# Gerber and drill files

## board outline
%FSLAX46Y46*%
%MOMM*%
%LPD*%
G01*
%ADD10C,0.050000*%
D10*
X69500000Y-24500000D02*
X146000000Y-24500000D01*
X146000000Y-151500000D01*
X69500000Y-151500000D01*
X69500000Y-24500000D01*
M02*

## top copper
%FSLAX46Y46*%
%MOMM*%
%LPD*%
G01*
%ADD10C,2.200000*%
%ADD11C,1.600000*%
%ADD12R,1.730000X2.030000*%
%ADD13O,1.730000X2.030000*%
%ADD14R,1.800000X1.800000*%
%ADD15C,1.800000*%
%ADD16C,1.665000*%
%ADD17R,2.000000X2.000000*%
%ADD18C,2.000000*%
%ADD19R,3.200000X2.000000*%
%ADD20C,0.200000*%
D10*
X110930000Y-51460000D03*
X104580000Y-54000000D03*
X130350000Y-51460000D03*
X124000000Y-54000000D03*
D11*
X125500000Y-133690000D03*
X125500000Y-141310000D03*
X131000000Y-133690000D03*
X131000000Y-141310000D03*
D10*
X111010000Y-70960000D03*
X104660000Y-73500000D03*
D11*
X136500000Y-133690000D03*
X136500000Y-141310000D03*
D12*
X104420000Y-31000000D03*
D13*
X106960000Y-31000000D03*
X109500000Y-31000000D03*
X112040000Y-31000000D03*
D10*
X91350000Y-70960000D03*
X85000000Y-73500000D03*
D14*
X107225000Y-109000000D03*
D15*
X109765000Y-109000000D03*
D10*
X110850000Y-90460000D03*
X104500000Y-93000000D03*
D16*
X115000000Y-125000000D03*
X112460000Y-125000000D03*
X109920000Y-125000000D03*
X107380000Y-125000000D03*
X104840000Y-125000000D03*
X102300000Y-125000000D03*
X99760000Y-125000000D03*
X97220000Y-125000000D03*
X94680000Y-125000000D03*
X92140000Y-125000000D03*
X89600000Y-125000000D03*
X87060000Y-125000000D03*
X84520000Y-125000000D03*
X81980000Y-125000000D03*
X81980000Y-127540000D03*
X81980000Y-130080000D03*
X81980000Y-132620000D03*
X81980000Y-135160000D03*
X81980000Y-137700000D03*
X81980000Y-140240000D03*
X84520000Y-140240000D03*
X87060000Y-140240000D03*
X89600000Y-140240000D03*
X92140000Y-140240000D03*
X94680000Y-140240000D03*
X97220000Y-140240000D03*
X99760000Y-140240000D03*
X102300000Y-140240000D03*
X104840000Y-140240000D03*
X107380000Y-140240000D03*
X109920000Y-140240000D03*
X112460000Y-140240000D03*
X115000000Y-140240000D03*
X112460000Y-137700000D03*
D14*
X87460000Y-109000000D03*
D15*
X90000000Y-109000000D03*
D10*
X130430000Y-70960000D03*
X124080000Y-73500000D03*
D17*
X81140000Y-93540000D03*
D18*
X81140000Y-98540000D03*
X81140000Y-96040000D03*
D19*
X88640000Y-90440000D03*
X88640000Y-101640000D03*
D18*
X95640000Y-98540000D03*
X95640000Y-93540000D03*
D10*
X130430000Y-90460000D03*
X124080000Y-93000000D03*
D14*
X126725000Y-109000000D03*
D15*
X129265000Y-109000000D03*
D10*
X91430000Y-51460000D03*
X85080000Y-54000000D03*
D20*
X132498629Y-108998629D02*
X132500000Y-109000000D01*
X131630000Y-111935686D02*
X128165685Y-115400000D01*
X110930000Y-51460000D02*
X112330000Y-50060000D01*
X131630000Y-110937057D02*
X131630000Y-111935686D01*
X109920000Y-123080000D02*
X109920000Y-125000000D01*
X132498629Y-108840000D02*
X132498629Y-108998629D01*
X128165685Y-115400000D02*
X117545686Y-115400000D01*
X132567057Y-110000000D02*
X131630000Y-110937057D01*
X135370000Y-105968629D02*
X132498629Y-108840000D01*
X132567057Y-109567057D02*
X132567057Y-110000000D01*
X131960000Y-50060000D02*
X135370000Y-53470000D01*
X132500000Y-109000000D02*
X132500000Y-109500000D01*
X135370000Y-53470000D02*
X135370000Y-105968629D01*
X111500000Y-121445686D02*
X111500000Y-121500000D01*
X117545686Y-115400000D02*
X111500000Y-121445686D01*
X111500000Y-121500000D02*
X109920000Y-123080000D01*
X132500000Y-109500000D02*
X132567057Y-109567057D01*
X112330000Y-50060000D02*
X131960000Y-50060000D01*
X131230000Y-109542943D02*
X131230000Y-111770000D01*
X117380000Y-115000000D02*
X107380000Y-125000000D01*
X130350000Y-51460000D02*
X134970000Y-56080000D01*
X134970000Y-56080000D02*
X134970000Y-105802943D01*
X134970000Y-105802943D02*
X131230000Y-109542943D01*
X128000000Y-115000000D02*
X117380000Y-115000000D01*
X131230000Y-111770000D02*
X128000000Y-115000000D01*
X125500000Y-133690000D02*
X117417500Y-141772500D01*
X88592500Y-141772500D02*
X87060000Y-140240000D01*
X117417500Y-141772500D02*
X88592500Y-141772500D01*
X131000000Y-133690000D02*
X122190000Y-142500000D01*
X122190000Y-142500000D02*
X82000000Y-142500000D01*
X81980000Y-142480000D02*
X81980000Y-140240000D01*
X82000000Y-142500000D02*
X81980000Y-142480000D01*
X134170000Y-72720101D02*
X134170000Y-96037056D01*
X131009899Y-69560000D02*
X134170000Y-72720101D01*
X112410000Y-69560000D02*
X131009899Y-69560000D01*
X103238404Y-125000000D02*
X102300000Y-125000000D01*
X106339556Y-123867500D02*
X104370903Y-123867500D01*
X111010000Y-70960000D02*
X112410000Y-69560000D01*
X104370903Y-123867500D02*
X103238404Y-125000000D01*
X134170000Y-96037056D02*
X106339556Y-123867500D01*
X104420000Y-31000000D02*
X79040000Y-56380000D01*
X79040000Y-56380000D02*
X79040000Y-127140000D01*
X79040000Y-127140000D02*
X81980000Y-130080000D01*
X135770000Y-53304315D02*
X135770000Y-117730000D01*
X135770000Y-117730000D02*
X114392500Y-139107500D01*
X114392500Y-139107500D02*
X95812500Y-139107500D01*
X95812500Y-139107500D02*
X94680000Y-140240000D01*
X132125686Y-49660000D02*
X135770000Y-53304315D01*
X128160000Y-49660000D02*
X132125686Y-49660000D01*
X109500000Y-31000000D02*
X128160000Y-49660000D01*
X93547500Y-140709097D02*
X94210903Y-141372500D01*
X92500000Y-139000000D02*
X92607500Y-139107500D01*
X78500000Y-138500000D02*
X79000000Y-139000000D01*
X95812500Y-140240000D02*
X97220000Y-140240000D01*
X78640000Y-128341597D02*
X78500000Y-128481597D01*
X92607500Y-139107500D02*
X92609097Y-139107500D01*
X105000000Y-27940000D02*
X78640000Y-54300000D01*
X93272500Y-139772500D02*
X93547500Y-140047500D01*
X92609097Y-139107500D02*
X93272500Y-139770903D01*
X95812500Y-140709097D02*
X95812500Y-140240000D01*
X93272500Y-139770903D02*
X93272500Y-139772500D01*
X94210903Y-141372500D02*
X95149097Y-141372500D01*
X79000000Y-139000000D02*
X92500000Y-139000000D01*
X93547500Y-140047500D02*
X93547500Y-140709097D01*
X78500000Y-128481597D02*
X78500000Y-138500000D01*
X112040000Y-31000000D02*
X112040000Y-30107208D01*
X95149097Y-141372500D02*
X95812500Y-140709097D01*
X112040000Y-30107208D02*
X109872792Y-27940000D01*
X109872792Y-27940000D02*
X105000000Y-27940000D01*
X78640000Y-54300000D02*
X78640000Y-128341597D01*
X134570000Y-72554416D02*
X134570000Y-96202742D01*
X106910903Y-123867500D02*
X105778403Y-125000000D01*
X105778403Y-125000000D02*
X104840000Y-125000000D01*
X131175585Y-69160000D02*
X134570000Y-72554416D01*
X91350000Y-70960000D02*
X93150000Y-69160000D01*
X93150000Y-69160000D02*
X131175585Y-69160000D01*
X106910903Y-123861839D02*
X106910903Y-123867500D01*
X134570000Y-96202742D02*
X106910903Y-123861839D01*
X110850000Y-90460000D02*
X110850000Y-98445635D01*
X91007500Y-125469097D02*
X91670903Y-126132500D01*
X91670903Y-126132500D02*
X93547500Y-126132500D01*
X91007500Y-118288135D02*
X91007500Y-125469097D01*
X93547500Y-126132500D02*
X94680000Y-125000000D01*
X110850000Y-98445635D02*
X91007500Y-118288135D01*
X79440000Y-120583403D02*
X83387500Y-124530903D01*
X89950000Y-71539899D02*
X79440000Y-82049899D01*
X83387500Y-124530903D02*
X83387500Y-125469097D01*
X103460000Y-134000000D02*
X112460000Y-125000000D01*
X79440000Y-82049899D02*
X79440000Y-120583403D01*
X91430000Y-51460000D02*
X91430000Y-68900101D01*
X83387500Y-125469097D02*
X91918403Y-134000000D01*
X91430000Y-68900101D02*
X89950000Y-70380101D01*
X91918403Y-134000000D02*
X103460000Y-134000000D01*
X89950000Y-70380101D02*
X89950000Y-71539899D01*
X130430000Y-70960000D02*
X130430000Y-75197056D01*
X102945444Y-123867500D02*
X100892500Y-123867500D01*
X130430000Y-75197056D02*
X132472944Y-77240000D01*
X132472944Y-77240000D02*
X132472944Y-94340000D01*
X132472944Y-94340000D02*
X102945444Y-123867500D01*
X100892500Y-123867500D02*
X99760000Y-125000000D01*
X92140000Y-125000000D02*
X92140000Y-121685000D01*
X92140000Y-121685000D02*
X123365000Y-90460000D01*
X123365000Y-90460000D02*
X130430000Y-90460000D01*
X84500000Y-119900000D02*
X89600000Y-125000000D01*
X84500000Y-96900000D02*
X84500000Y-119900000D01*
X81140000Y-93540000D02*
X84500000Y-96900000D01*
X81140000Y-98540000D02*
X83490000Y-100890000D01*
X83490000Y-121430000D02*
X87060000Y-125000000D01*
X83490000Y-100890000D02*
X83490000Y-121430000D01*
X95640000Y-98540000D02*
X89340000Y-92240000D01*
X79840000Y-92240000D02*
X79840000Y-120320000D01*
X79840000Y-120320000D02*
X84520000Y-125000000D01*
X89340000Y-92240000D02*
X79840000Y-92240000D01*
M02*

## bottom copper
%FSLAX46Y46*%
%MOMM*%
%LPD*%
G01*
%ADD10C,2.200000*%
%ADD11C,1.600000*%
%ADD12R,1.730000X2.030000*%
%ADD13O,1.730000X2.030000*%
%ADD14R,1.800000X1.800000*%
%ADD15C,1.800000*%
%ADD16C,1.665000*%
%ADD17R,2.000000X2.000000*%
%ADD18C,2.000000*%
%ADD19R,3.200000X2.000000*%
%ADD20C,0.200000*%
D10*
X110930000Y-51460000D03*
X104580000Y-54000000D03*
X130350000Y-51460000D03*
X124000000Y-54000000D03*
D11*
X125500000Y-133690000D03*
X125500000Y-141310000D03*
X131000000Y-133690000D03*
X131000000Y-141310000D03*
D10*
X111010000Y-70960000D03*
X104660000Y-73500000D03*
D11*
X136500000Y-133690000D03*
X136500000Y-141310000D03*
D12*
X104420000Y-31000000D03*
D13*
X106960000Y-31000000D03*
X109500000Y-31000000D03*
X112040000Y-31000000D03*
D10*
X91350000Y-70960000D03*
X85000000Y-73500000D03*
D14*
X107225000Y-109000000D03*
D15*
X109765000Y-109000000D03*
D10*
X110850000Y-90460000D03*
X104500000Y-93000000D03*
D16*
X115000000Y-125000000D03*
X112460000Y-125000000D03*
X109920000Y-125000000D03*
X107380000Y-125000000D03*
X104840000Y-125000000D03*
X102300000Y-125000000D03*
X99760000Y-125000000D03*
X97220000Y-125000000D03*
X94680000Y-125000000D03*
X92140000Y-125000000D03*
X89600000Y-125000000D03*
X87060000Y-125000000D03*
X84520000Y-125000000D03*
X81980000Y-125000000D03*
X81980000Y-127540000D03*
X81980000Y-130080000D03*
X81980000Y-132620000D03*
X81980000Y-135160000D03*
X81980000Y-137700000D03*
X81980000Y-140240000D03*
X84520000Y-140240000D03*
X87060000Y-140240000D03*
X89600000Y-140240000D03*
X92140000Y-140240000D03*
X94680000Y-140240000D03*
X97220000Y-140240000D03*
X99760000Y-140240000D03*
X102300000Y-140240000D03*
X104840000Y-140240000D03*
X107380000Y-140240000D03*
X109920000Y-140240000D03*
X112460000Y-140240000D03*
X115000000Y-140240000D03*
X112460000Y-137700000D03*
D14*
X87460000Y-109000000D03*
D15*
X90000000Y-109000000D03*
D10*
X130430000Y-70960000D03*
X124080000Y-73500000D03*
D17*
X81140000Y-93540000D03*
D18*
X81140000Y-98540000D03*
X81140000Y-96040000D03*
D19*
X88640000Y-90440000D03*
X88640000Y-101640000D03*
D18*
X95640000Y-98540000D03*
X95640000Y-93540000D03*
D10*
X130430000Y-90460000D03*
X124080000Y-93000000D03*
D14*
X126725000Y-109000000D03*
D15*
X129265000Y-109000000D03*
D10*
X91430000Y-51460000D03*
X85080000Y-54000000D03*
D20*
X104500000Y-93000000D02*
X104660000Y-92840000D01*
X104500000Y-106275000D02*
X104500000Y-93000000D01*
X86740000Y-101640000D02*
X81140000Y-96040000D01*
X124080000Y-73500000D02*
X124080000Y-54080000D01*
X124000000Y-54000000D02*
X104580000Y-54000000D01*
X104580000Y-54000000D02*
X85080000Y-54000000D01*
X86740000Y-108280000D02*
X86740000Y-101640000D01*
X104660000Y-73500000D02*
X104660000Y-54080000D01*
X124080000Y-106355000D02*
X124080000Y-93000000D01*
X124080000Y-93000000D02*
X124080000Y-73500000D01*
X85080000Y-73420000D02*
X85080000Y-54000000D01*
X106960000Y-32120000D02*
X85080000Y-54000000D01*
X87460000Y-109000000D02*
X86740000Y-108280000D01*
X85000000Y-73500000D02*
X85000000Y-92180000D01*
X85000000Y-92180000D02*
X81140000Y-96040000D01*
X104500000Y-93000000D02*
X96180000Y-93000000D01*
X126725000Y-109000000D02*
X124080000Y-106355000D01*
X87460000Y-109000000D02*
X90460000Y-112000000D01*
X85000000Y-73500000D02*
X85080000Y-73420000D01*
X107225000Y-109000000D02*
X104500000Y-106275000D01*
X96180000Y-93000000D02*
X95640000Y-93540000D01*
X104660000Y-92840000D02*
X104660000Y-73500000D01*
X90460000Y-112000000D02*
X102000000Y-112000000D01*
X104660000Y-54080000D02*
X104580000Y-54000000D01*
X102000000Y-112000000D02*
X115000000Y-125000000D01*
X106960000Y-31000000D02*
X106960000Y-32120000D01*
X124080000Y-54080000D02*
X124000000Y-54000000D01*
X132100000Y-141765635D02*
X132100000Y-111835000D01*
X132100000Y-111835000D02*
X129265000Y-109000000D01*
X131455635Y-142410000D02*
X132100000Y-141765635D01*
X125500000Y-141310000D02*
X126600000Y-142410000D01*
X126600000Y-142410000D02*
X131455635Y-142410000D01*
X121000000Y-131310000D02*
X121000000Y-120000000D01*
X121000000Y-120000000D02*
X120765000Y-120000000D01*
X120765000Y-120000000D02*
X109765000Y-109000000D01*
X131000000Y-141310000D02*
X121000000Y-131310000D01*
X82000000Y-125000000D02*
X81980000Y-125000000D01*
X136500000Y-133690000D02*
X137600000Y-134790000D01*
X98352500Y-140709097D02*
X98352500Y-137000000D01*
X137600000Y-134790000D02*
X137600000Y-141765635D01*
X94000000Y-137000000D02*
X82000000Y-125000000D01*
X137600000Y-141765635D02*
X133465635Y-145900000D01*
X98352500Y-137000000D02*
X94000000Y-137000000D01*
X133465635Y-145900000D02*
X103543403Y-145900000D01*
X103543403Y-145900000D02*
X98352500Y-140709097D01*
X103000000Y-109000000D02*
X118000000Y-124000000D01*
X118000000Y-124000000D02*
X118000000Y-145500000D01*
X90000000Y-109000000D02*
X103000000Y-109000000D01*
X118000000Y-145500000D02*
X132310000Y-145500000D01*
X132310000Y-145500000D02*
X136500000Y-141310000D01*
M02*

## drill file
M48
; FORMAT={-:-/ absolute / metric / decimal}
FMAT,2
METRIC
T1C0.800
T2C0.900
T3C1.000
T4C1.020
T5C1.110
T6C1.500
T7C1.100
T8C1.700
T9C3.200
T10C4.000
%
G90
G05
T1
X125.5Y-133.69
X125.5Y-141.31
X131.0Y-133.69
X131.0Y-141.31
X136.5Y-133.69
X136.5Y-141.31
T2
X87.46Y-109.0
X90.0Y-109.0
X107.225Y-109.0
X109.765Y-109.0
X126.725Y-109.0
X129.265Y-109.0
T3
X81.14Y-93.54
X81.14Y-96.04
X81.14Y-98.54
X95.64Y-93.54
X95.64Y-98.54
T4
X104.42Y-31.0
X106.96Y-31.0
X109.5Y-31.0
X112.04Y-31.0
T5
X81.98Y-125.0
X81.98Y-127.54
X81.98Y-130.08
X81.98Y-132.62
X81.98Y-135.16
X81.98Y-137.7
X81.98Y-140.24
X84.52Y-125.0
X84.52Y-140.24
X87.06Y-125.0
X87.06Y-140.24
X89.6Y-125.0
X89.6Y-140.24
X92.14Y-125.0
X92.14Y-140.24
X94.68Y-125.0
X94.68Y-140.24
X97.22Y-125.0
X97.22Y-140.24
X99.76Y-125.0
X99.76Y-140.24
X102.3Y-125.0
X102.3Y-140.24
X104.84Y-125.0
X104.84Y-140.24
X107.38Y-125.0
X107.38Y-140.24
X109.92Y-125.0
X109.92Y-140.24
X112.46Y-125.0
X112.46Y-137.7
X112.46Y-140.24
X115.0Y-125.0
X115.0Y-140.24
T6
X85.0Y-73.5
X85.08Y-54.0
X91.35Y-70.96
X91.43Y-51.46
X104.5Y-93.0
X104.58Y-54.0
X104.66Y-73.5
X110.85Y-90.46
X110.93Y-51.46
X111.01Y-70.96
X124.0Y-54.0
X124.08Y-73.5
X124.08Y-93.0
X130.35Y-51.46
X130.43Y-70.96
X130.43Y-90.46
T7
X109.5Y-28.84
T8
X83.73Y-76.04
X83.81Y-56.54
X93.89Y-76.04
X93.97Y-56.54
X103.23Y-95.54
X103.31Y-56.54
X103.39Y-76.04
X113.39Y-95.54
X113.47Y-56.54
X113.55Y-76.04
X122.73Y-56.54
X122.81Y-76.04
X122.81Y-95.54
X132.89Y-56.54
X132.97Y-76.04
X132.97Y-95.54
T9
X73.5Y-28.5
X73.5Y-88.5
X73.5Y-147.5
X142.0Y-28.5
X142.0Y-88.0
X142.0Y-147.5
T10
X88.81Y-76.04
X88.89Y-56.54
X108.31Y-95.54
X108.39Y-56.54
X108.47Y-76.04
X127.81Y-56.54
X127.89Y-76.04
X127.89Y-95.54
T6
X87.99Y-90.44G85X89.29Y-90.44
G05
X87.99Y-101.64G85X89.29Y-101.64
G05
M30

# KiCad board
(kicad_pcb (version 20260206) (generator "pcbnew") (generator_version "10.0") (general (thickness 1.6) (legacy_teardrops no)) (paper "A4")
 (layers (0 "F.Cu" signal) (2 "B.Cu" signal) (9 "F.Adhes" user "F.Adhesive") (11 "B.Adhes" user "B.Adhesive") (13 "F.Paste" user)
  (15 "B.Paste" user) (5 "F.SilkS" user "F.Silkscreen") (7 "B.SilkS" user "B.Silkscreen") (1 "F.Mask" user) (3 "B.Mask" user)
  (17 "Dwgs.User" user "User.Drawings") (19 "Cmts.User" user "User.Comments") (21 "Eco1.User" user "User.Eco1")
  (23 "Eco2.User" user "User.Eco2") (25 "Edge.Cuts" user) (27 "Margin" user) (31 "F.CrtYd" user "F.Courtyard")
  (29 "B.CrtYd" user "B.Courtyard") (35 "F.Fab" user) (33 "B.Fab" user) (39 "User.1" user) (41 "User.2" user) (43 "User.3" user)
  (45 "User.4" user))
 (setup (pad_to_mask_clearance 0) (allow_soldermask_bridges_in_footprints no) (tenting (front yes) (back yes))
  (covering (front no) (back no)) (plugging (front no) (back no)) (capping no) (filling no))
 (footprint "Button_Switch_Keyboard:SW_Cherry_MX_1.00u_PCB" (layer "F.Cu") (at 110.93 51.46)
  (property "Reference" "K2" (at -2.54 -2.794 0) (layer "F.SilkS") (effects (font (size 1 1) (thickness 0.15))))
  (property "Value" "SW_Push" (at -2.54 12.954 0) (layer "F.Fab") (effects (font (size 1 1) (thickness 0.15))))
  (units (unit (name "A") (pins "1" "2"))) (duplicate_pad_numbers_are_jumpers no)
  (pad "" np_thru_hole circle (at -7.62 5.08) (size 1.7 1.7) (drill 1.7) (layers "*.Cu" "*.Mask"))
  (pad "" np_thru_hole circle (at -2.54 5.08) (size 4 4) (drill 4) (layers "*.Cu" "*.Mask"))
  (pad "" np_thru_hole circle (at 2.54 5.08) (size 1.7 1.7) (drill 1.7) (layers "*.Cu" "*.Mask"))
  (pad "1" thru_hole circle (at 0 0) (size 2.2 2.2) (drill 1.5) (layers "*.Cu" "*.Mask") (remove_unused_layers no) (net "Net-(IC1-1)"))
  (pad "2" thru_hole circle (at -6.35 2.54) (size 2.2 2.2) (drill 1.5) (layers "*.Cu" "*.Mask") (remove_unused_layers no) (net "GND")))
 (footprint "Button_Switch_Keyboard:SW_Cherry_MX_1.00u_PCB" (layer "F.Cu") (at 130.35 51.46)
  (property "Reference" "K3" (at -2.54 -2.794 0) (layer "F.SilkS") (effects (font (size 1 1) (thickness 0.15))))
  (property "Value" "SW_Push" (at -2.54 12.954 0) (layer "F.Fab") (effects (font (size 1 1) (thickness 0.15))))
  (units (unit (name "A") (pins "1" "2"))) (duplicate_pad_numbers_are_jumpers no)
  (pad "" np_thru_hole circle (at -7.62 5.08) (size 1.7 1.7) (drill 1.7) (layers "*.Cu" "*.Mask"))
  (pad "" np_thru_hole circle (at -2.54 5.08) (size 4 4) (drill 4) (layers "*.Cu" "*.Mask"))
  (pad "" np_thru_hole circle (at 2.54 5.08) (size 1.7 1.7) (drill 1.7) (layers "*.Cu" "*.Mask"))
  (pad "1" thru_hole circle (at 0 0) (size 2.2 2.2) (drill 1.5) (layers "*.Cu" "*.Mask") (remove_unused_layers no) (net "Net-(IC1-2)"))
  (pad "2" thru_hole circle (at -6.35 2.54) (size 2.2 2.2) (drill 1.5) (layers "*.Cu" "*.Mask") (remove_unused_layers no) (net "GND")))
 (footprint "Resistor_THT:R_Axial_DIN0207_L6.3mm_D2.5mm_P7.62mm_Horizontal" (layer "F.Cu") (at 125.5 133.69 -90)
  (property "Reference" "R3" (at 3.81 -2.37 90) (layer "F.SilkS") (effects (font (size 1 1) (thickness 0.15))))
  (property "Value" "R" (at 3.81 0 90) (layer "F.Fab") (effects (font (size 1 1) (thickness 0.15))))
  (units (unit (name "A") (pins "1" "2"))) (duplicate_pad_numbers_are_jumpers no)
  (pad "1" thru_hole circle (at 0 0 270) (size 1.6 1.6) (drill 0.8) (layers "*.Cu" "*.Mask") (remove_unused_layers no)
   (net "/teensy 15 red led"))
  (pad "2" thru_hole circle (at 7.62 0 270) (size 1.6 1.6) (drill 0.8) (layers "*.Cu" "*.Mask") (remove_unused_layers no) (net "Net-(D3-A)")))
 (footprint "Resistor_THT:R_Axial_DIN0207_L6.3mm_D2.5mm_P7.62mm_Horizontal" (layer "F.Cu") (at 131 133.69 -90)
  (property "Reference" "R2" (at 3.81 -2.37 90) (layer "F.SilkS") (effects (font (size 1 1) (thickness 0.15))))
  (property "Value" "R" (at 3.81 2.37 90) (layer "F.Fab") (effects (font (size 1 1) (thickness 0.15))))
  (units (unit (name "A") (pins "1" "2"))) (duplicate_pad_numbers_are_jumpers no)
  (pad "1" thru_hole circle (at 0 0 270) (size 1.6 1.6) (drill 0.8) (layers "*.Cu" "*.Mask") (remove_unused_layers no) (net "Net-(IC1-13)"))
  (pad "2" thru_hole circle (at 7.62 0 270) (size 1.6 1.6) (drill 0.8) (layers "*.Cu" "*.Mask") (remove_unused_layers no) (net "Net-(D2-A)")))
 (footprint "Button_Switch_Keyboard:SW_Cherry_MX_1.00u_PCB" (layer "F.Cu") (at 111.01 70.96)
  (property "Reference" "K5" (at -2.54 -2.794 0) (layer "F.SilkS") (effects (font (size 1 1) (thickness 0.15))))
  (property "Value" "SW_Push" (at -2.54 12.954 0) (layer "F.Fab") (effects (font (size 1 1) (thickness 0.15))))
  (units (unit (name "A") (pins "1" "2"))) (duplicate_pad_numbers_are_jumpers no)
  (pad "" np_thru_hole circle (at -7.62 5.08) (size 1.7 1.7) (drill 1.7) (layers "*.Cu" "*.Mask"))
  (pad "" np_thru_hole circle (at -2.54 5.08) (size 4 4) (drill 4) (layers "*.Cu" "*.Mask"))
  (pad "" np_thru_hole circle (at 2.54 5.08) (size 1.7 1.7) (drill 1.7) (layers "*.Cu" "*.Mask"))
  (pad "1" thru_hole circle (at 0 0) (size 2.2 2.2) (drill 1.5) (layers "*.Cu" "*.Mask") (remove_unused_layers no) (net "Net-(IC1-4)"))
  (pad "2" thru_hole circle (at -6.35 2.54) (size 2.2 2.2) (drill 1.5) (layers "*.Cu" "*.Mask") (remove_unused_layers no) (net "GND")))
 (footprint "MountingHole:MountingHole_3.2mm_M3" (layer "F.Cu") (at 73.5 88.5)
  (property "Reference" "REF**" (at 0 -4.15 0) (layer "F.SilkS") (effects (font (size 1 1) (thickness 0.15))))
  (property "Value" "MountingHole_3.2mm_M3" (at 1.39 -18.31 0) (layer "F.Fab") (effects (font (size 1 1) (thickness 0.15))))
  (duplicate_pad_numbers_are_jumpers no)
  (pad "" np_thru_hole circle (at 0 0) (size 3.2 3.2) (drill 3.2) (layers "*.Cu" "*.Mask")))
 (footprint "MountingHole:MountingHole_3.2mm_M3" (layer "F.Cu") (at 142 147.5)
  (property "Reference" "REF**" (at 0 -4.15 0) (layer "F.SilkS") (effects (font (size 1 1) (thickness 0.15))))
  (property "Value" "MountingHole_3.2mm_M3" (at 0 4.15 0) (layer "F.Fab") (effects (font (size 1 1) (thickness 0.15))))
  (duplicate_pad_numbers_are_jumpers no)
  (pad "" np_thru_hole circle (at 0 0) (size 3.2 3.2) (drill 3.2) (layers "*.Cu" "*.Mask")))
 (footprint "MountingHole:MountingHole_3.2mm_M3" (layer "F.Cu") (at 142 28.5)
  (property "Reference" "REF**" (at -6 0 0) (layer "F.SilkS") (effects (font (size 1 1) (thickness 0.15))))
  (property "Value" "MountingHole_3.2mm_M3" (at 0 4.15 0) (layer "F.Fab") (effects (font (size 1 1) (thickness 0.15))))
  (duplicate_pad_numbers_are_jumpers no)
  (pad "" np_thru_hole circle (at 0 0) (size 3.2 3.2) (drill 3.2) (layers "*.Cu" "*.Mask")))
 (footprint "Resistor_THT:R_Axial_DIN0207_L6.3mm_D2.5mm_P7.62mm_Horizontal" (layer "F.Cu") (at 136.5 133.69 -90)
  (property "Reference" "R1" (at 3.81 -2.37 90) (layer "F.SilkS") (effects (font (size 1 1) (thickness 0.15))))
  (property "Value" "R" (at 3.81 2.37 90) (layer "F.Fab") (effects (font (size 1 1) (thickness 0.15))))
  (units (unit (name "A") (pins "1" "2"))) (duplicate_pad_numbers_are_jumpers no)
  (pad "1" thru_hole circle (at 0 0 270) (size 1.6 1.6) (drill 0.8) (layers "*.Cu" "*.Mask") (remove_unused_layers no) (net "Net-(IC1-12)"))
  (pad "2" thru_hole circle (at 7.62 0 270) (size 1.6 1.6) (drill 0.8) (layers "*.Cu" "*.Mask") (remove_unused_layers no) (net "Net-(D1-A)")))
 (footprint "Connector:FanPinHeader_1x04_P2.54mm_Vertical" (layer "F.Cu") (at 104.42 31)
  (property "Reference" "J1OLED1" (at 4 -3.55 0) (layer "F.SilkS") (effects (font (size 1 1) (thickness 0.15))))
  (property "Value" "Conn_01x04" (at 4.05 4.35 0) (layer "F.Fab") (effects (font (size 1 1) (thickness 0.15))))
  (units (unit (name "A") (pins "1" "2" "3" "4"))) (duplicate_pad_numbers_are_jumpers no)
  (pad "" np_thru_hole circle (at 5.08 -2.16 90) (size 1.1 1.1) (drill 1.1) (layers "*.Cu" "*.Mask"))
  (pad "1" thru_hole rect (at 0 0 90) (size 2.03 1.73) (drill 1.02) (layers "*.Cu" "*.Mask") (remove_unused_layers no) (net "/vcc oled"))
  (pad "2" thru_hole oval (at 2.54 0 90) (size 2.03 1.73) (drill 1.02) (layers "*.Cu" "*.Mask") (remove_unused_layers no) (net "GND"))
  (pad "3" thru_hole oval (at 5.08 0 90) (size 2.03 1.73) (drill 1.02) (layers "*.Cu" "*.Mask") (remove_unused_layers no) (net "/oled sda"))
  (pad "4" thru_hole oval (at 7.62 0 90) (size 2.03 1.73) (drill 1.02) (layers "*.Cu" "*.Mask") (remove_unused_layers no) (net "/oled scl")))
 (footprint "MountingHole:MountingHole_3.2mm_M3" (layer "F.Cu") (at 73.5 147.5)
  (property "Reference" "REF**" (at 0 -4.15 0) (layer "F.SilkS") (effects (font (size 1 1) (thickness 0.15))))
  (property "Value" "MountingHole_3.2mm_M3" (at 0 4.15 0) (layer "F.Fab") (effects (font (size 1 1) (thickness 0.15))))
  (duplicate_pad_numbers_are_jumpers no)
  (pad "" np_thru_hole circle (at 0 0) (size 3.2 3.2) (drill 3.2) (layers "*.Cu" "*.Mask")))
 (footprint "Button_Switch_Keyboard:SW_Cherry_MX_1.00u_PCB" (layer "F.Cu") (at 91.35 70.96)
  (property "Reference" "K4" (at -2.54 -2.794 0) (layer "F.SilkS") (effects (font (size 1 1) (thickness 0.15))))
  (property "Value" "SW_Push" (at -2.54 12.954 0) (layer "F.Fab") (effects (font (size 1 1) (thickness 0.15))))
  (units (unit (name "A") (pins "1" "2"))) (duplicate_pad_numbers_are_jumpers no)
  (pad "" np_thru_hole circle (at -7.62 5.08) (size 1.7 1.7) (drill 1.7) (layers "*.Cu" "*.Mask"))
  (pad "" np_thru_hole circle (at -2.54 5.08) (size 4 4) (drill 4) (layers "*.Cu" "*.Mask"))
  (pad "" np_thru_hole circle (at 2.54 5.08) (size 1.7 1.7) (drill 1.7) (layers "*.Cu" "*.Mask"))
  (pad "1" thru_hole circle (at 0 0) (size 2.2 2.2) (drill 1.5) (layers "*.Cu" "*.Mask") (remove_unused_layers no) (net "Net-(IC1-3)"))
  (pad "2" thru_hole circle (at -6.35 2.54) (size 2.2 2.2) (drill 1.5) (layers "*.Cu" "*.Mask") (remove_unused_layers no) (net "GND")))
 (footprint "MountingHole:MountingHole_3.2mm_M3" (layer "F.Cu") (at 73.5 28.5)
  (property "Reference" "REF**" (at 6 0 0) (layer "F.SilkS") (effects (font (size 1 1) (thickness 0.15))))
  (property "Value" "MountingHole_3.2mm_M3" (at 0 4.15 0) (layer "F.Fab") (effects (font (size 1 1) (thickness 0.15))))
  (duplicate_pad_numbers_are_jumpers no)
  (pad "" np_thru_hole circle (at 0 0) (size 3.2 3.2) (drill 3.2) (layers "*.Cu" "*.Mask")))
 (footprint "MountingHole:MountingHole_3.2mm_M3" (layer "F.Cu") (at 142 88)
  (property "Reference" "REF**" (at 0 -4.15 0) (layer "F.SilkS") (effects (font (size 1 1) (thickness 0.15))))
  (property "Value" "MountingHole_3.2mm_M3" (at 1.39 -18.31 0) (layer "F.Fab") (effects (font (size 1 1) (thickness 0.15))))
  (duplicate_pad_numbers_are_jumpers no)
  (pad "" np_thru_hole circle (at 0 0) (size 3.2 3.2) (drill 3.2) (layers "*.Cu" "*.Mask")))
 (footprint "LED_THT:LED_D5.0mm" (layer "F.Cu") (at 107.225 109)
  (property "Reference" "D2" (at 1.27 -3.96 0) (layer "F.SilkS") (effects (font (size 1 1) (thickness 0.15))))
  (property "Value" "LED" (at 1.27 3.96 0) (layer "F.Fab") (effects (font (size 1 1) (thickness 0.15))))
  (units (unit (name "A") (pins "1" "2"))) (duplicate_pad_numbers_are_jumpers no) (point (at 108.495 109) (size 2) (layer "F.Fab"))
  (pad "1" thru_hole rect (at 0 0) (size 1.8 1.8) (drill 0.9) (layers "*.Cu" "*.Mask") (remove_unused_layers no) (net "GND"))
  (pad "2" thru_hole circle (at 2.54 0) (size 1.8 1.8) (drill 0.9) (layers "*.Cu" "*.Mask") (remove_unused_layers no) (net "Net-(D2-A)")))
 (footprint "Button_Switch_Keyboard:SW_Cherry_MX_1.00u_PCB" (layer "F.Cu") (at 110.85 90.46)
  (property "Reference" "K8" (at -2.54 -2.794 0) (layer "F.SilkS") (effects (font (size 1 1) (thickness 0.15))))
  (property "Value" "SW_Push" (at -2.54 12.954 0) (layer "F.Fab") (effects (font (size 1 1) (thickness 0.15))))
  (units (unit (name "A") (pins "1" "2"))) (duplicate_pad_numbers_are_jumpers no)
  (pad "" np_thru_hole circle (at -7.62 5.08) (size 1.7 1.7) (drill 1.7) (layers "*.Cu" "*.Mask"))
  (pad "" np_thru_hole circle (at -2.54 5.08) (size 4 4) (drill 4) (layers "*.Cu" "*.Mask"))
  (pad "" np_thru_hole circle (at 2.54 5.08) (size 1.7 1.7) (drill 1.7) (layers "*.Cu" "*.Mask"))
  (pad "1" thru_hole circle (at 0 0) (size 2.2 2.2) (drill 1.5) (layers "*.Cu" "*.Mask") (remove_unused_layers no) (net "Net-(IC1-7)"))
  (pad "2" thru_hole circle (at -6.35 2.54) (size 2.2 2.2) (drill 1.5) (layers "*.Cu" "*.Mask") (remove_unused_layers no) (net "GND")))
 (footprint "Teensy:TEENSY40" (layer "F.Cu") (at 115 125 180)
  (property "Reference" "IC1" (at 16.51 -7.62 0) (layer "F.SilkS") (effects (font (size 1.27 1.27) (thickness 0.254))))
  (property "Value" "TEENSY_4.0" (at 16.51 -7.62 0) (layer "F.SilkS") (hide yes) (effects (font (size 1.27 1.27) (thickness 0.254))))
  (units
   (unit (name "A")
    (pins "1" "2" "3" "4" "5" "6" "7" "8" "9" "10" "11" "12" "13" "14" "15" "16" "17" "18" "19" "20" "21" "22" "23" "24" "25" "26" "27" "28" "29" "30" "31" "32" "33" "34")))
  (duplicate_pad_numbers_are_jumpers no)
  (pad "1" thru_hole circle (at 0 0 180) (size 1.665 1.665) (drill 1.11) (layers "*.Cu" "*.Mask") (remove_unused_layers no) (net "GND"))
  (pad "2" thru_hole circle (at 2.54 0 180) (size 1.665 1.665) (drill 1.11) (layers "*.Cu" "*.Mask") (remove_unused_layers no)
   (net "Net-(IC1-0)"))
  (pad "3" thru_hole circle (at 5.08 0 180) (size 1.665 1.665) (drill 1.11) (layers "*.Cu" "*.Mask") (remove_unused_layers no)
   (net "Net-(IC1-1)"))
  (pad "4" thru_hole circle (at 7.62 0 180) (size 1.665 1.665) (drill 1.11) (layers "*.Cu" "*.Mask") (remove_unused_layers no)
   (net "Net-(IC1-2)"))
  (pad "5" thru_hole circle (at 10.16 0 180) (size 1.665 1.665) (drill 1.11) (layers "*.Cu" "*.Mask") (remove_unused_layers no)
   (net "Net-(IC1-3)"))
  (pad "6" thru_hole circle (at 12.7 0 180) (size 1.665 1.665) (drill 1.11) (layers "*.Cu" "*.Mask") (remove_unused_layers no)
   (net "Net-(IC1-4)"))
  (pad "7" thru_hole circle (at 15.24 0 180) (size 1.665 1.665) (drill 1.11) (layers "*.Cu" "*.Mask") (remove_unused_layers no)
   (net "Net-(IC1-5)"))
  (pad "8" thru_hole circle (at 17.78 0 180) (size 1.665 1.665) (drill 1.11) (layers "*.Cu" "*.Mask") (remove_unused_layers no)
   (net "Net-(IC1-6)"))
  (pad "9" thru_hole circle (at 20.32 0 180) (size 1.665 1.665) (drill 1.11) (layers "*.Cu" "*.Mask") (remove_unused_layers no)
   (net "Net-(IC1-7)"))
  (pad "10" thru_hole circle (at 22.86 0 180) (size 1.665 1.665) (drill 1.11) (layers "*.Cu" "*.Mask") (remove_unused_layers no)
   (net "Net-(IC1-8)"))
  (pad "11" thru_hole circle (at 25.4 0 180) (size 1.665 1.665) (drill 1.11) (layers "*.Cu" "*.Mask") (remove_unused_layers no)
   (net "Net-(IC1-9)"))
  (pad "12" thru_hole circle (at 27.94 0 180) (size 1.665 1.665) (drill 1.11) (layers "*.Cu" "*.Mask") (remove_unused_layers no)
   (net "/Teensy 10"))
  (pad "13" thru_hole circle (at 30.48 0 180) (size 1.665 1.665) (drill 1.11) (layers "*.Cu" "*.Mask") (remove_unused_layers no)
   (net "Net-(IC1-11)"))
  (pad "14" thru_hole circle (at 33.02 0 180) (size 1.665 1.665) (drill 1.11) (layers "*.Cu" "*.Mask") (remove_unused_layers no)
   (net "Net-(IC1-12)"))
  (pad "15" thru_hole circle (at 33.02 -2.54 180) (size 1.665 1.665) (drill 1.11) (layers "*.Cu" "*.Mask") (remove_unused_layers no)
   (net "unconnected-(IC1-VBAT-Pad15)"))
  (pad "16" thru_hole circle (at 33.02 -5.08 180) (size 1.665 1.665) (drill 1.11) (layers "*.Cu" "*.Mask") (remove_unused_layers no)
   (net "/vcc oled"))
  (pad "17" thru_hole circle (at 33.02 -7.62 180) (size 1.665 1.665) (drill 1.11) (layers "*.Cu" "*.Mask") (remove_unused_layers no)
   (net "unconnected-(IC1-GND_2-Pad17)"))
  (pad "18" thru_hole circle (at 33.02 -10.16 180) (size 1.665 1.665) (drill 1.11) (layers "*.Cu" "*.Mask") (remove_unused_layers no)
   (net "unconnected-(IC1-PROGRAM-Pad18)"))
  (pad "19" thru_hole circle (at 33.02 -12.7 180) (size 1.665 1.665) (drill 1.11) (layers "*.Cu" "*.Mask") (remove_unused_layers no)
   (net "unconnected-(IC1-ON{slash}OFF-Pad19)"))
  (pad "20" thru_hole circle (at 33.02 -15.24 180) (size 1.665 1.665) (drill 1.11) (layers "*.Cu" "*.Mask") (remove_unused_layers no)
   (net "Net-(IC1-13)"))
  (pad "21" thru_hole circle (at 30.48 -15.24 180) (size 1.665 1.665) (drill 1.11) (layers "*.Cu" "*.Mask") (remove_unused_layers no)
   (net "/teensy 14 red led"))
  (pad "22" thru_hole circle (at 27.94 -15.24 180) (size 1.665 1.665) (drill 1.11) (layers "*.Cu" "*.Mask") (remove_unused_layers no)
   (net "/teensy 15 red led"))
  (pad "23" thru_hole circle (at 25.4 -15.24 180) (size 1.665 1.665) (drill 1.11) (layers "*.Cu" "*.Mask") (remove_unused_layers no)
   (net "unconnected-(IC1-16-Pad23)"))
  (pad "24" thru_hole circle (at 22.86 -15.24 180) (size 1.665 1.665) (drill 1.11) (layers "*.Cu" "*.Mask") (remove_unused_layers no)
   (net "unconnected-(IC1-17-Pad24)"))
  (pad "25" thru_hole circle (at 20.32 -15.24 180) (size 1.665 1.665) (drill 1.11) (layers "*.Cu" "*.Mask") (remove_unused_layers no)
   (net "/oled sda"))
  (pad "26" thru_hole circle (at 17.78 -15.24 180) (size 1.665 1.665) (drill 1.11) (layers "*.Cu" "*.Mask") (remove_unused_layers no)
   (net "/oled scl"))
  (pad "27" thru_hole circle (at 15.24 -15.24 180) (size 1.665 1.665) (drill 1.11) (layers "*.Cu" "*.Mask") (remove_unused_layers no)
   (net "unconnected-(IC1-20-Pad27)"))
  (pad "28" thru_hole circle (at 12.7 -15.24 180) (size 1.665 1.665) (drill 1.11) (layers "*.Cu" "*.Mask") (remove_unused_layers no)
   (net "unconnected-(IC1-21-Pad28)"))
  (pad "29" thru_hole circle (at 10.16 -15.24 180) (size 1.665 1.665) (drill 1.11) (layers "*.Cu" "*.Mask") (remove_unused_layers no)
   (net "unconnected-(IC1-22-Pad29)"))
  (pad "30" thru_hole circle (at 7.62 -15.24 180) (size 1.665 1.665) (drill 1.11) (layers "*.Cu" "*.Mask") (remove_unused_layers no)
   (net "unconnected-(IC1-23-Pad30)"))
  (pad "31" thru_hole circle (at 5.08 -15.24 180) (size 1.665 1.665) (drill 1.11) (layers "*.Cu" "*.Mask") (remove_unused_layers no)
   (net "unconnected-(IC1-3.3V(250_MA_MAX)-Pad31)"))
  (pad "32" thru_hole circle (at 2.54 -15.24 180) (size 1.665 1.665) (drill 1.11) (layers "*.Cu" "*.Mask") (remove_unused_layers no)
   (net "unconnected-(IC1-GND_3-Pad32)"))
  (pad "33" thru_hole circle (at 0 -15.24 180) (size 1.665 1.665) (drill 1.11) (layers "*.Cu" "*.Mask") (remove_unused_layers no)
   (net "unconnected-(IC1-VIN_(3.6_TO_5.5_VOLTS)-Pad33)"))
  (pad "34" thru_hole circle (at 2.54 -12.7 180) (size 1.665 1.665) (drill 1.11) (layers "*.Cu" "*.Mask") (remove_unused_layers no)
   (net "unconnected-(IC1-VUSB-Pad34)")))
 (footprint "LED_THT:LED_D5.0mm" (layer "F.Cu") (at 87.46 109)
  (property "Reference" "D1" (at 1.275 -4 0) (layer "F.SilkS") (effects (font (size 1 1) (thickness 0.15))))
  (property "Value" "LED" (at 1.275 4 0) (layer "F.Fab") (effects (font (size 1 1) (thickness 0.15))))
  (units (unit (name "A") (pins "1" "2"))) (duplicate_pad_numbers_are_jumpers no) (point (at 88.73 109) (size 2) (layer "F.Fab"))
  (pad "1" thru_hole rect (at 0 0) (size 1.8 1.8) (drill 0.9) (layers "*.Cu" "*.Mask") (remove_unused_layers no) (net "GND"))
  (pad "2" thru_hole circle (at 2.54 0) (size 1.8 1.8) (drill 0.9) (layers "*.Cu" "*.Mask") (remove_unused_layers no) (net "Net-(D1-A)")))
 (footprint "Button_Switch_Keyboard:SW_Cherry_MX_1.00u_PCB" (layer "F.Cu") (at 130.43 70.96)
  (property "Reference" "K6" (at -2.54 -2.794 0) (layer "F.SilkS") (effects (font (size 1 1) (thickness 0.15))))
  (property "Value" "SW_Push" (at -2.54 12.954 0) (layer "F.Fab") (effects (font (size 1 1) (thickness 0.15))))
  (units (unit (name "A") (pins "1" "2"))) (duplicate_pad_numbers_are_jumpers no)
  (pad "" np_thru_hole circle (at -7.62 5.08) (size 1.7 1.7) (drill 1.7) (layers "*.Cu" "*.Mask"))
  (pad "" np_thru_hole circle (at -2.54 5.08) (size 4 4) (drill 4) (layers "*.Cu" "*.Mask"))
  (pad "" np_thru_hole circle (at 2.54 5.08) (size 1.7 1.7) (drill 1.7) (layers "*.Cu" "*.Mask"))
  (pad "1" thru_hole circle (at 0 0) (size 2.2 2.2) (drill 1.5) (layers "*.Cu" "*.Mask") (remove_unused_layers no) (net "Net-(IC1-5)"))
  (pad "2" thru_hole circle (at -6.35 2.54) (size 2.2 2.2) (drill 1.5) (layers "*.Cu" "*.Mask") (remove_unused_layers no) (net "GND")))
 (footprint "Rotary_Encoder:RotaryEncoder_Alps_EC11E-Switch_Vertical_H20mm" (layer "F.Cu") (at 81.14 93.54)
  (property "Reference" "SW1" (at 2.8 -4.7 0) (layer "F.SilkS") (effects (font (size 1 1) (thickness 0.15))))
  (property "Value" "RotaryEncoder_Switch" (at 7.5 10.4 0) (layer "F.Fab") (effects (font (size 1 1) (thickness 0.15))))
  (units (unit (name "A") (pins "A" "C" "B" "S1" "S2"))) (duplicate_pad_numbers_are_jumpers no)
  (pad "A" thru_hole rect (at 0 0) (size 2 2) (drill 1) (layers "*.Cu" "*.Mask") (remove_unused_layers no) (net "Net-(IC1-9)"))
  (pad "B" thru_hole circle (at 0 5) (size 2 2) (drill 1) (layers "*.Cu" "*.Mask") (remove_unused_layers no) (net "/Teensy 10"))
  (pad "C" thru_hole circle (at 0 2.5) (size 2 2) (drill 1) (layers "*.Cu" "*.Mask") (remove_unused_layers no) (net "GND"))
  (pad "MP" thru_hole rect (at 7.5 -3.1) (size 3.2 2) (drill oval 2.8 1.5) (layers "*.Cu" "*.Mask") (remove_unused_layers no))
  (pad "MP" thru_hole rect (at 7.5 8.1) (size 3.2 2) (drill oval 2.8 1.5) (layers "*.Cu" "*.Mask") (remove_unused_layers no))
  (pad "S1" thru_hole circle (at 14.5 5) (size 2 2) (drill 1) (layers "*.Cu" "*.Mask") (remove_unused_layers no) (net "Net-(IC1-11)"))
  (pad "S2" thru_hole circle (at 14.5 0) (size 2 2) (drill 1) (layers "*.Cu" "*.Mask") (remove_unused_layers no) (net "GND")))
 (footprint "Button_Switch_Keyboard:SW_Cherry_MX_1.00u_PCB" (layer "F.Cu") (at 130.43 90.46)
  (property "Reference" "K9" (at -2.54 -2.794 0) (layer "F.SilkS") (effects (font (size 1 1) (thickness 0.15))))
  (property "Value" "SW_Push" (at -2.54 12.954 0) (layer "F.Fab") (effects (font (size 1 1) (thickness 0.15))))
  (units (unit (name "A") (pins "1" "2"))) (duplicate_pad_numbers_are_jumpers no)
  (pad "" np_thru_hole circle (at -7.62 5.08) (size 1.7 1.7) (drill 1.7) (layers "*.Cu" "*.Mask"))
  (pad "" np_thru_hole circle (at -2.54 5.08) (size 4 4) (drill 4) (layers "*.Cu" "*.Mask"))
  (pad "" np_thru_hole circle (at 2.54 5.08) (size 1.7 1.7) (drill 1.7) (layers "*.Cu" "*.Mask"))
  (pad "1" thru_hole circle (at 0 0) (size 2.2 2.2) (drill 1.5) (layers "*.Cu" "*.Mask") (remove_unused_layers no) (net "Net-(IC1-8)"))
  (pad "2" thru_hole circle (at -6.35 2.54) (size 2.2 2.2) (drill 1.5) (layers "*.Cu" "*.Mask") (remove_unused_layers no) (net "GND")))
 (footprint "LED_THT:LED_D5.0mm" (layer "F.Cu") (at 126.725 109)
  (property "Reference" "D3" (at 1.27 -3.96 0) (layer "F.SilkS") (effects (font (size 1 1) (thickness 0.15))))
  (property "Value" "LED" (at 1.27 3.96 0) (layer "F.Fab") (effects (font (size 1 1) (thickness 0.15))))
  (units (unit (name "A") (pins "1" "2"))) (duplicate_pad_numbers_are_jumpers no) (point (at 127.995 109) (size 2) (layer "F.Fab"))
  (pad "1" thru_hole rect (at 0 0) (size 1.8 1.8) (drill 0.9) (layers "*.Cu" "*.Mask") (remove_unused_layers no) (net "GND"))
  (pad "2" thru_hole circle (at 2.54 0) (size 1.8 1.8) (drill 0.9) (layers "*.Cu" "*.Mask") (remove_unused_layers no) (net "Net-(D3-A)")))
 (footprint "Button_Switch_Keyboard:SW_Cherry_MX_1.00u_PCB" (layer "F.Cu") (at 91.43 51.46)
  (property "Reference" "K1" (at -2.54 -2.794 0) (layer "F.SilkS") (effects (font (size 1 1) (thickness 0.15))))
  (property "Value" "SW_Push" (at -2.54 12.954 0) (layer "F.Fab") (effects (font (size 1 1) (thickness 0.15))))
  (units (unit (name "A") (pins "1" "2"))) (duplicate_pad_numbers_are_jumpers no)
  (pad "" np_thru_hole circle (at -7.62 5.08) (size 1.7 1.7) (drill 1.7) (layers "*.Cu" "*.Mask"))
  (pad "" np_thru_hole circle (at -2.54 5.08) (size 4 4) (drill 4) (layers "*.Cu" "*.Mask"))
  (pad "" np_thru_hole circle (at 2.54 5.08) (size 1.7 1.7) (drill 1.7) (layers "*.Cu" "*.Mask"))
  (pad "1" thru_hole circle (at 0 0) (size 2.2 2.2) (drill 1.5) (layers "*.Cu" "*.Mask") (remove_unused_layers no) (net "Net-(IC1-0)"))
  (pad "2" thru_hole circle (at -6.35 2.54) (size 2.2 2.2) (drill 1.5) (layers "*.Cu" "*.Mask") (remove_unused_layers no) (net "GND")))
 (gr_rect (start 69.5 24.5) (end 146 151.5) (stroke (width 0.05) (type default)) (fill no) (layer "Edge.Cuts"))
 (segment (start 132.498629 108.998629) (end 132.5 109) (width 0.2) (layer "F.Cu") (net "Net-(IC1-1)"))
 (segment (start 131.63 111.935686) (end 128.165685 115.4) (width 0.2) (layer "F.Cu") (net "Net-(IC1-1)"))
 (segment (start 110.93 51.46) (end 112.33 50.06) (width 0.2) (layer "F.Cu") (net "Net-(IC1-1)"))
 (segment (start 131.63 110.937057) (end 131.63 111.935686) (width 0.2) (layer "F.Cu") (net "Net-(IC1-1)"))
 (segment (start 109.92 123.08) (end 109.92 125) (width 0.2) (layer "F.Cu") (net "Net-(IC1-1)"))
 (segment (start 132.498629 108.84) (end 132.498629 108.998629) (width 0.2) (layer "F.Cu") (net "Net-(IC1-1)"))
 (segment (start 128.165685 115.4) (end 117.545686 115.4) (width 0.2) (layer "F.Cu") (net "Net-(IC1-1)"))
 (segment (start 132.567057 110) (end 131.63 110.937057) (width 0.2) (layer "F.Cu") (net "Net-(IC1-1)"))
 (segment (start 135.37 105.968629) (end 132.498629 108.84) (width 0.2) (layer "F.Cu") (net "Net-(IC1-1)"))
 (segment (start 132.567057 109.567057) (end 132.567057 110) (width 0.2) (layer "F.Cu") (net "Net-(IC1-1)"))
 (segment (start 131.96 50.06) (end 135.37 53.47) (width 0.2) (layer "F.Cu") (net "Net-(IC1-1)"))
 (segment (start 132.5 109) (end 132.5 109.5) (width 0.2) (layer "F.Cu") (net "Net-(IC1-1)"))
 (segment (start 135.37 53.47) (end 135.37 105.968629) (width 0.2) (layer "F.Cu") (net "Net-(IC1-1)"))
 (segment (start 111.5 121.445686) (end 111.5 121.5) (width 0.2) (layer "F.Cu") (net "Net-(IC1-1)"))
 (segment (start 117.545686 115.4) (end 111.5 121.445686) (width 0.2) (layer "F.Cu") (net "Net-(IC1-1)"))
 (segment (start 111.5 121.5) (end 109.92 123.08) (width 0.2) (layer "F.Cu") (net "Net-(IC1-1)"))
 (segment (start 132.5 109.5) (end 132.567057 109.567057) (width 0.2) (layer "F.Cu") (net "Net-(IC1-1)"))
 (segment (start 112.33 50.06) (end 131.96 50.06) (width 0.2) (layer "F.Cu") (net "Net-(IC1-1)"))
 (segment (start 104.5 93) (end 104.66 92.84) (width 0.2) (layer "B.Cu") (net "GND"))
 (segment (start 104.5 106.275) (end 104.5 93) (width 0.2) (layer "B.Cu") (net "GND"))
 (segment (start 86.74 101.64) (end 81.14 96.04) (width 0.2) (layer "B.Cu") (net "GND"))
 (segment (start 124.08 73.5) (end 124.08 54.08) (width 0.2) (layer "B.Cu") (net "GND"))
 (segment (start 124 54) (end 104.58 54) (width 0.2) (layer "B.Cu") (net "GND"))
 (segment (start 104.58 54) (end 85.08 54) (width 0.2) (layer "B.Cu") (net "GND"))
 (segment (start 86.74 108.28) (end 86.74 101.64) (width 0.2) (layer "B.Cu") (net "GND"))
 (segment (start 104.66 73.5) (end 104.66 54.08) (width 0.2) (layer "B.Cu") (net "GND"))
 (segment (start 124.08 106.355) (end 124.08 93) (width 0.2) (layer "B.Cu") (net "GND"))
 (segment (start 124.08 93) (end 124.08 73.5) (width 0.2) (layer "B.Cu") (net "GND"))
 (segment (start 85.08 73.42) (end 85.08 54) (width 0.2) (layer "B.Cu") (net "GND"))
 (segment (start 106.96 32.12) (end 85.08 54) (width 0.2) (layer "B.Cu") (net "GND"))
 (segment (start 87.46 109) (end 86.74 108.28) (width 0.2) (layer "B.Cu") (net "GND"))
 (segment (start 85 73.5) (end 85 92.18) (width 0.2) (layer "B.Cu") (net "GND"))
 (segment (start 85 92.18) (end 81.14 96.04) (width 0.2) (layer "B.Cu") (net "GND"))
 (segment (start 104.5 93) (end 96.18 93) (width 0.2) (layer "B.Cu") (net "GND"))
 (segment (start 126.725 109) (end 124.08 106.355) (width 0.2) (layer "B.Cu") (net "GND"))
 (segment (start 87.46 109) (end 90.46 112) (width 0.2) (layer "B.Cu") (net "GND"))
 (segment (start 85 73.5) (end 85.08 73.42) (width 0.2) (layer "B.Cu") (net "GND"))
 (segment (start 107.225 109) (end 104.5 106.275) (width 0.2) (layer "B.Cu") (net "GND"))
 (segment (start 96.18 93) (end 95.64 93.54) (width 0.2) (layer "B.Cu") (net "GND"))
 (segment (start 104.66 92.84) (end 104.66 73.5) (width 0.2) (layer "B.Cu") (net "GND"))
 (segment (start 90.46 112) (end 102 112) (width 0.2) (layer "B.Cu") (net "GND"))
 (segment (start 104.66 54.08) (end 104.58 54) (width 0.2) (layer "B.Cu") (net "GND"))
 (segment (start 102 112) (end 115 125) (width 0.2) (layer "B.Cu") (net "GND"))
 (segment (start 106.96 31) (end 106.96 32.12) (width 0.2) (layer "B.Cu") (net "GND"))
 (segment (start 124.08 54.08) (end 124 54) (width 0.2) (layer "B.Cu") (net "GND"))
 (segment (start 131.23 109.542943) (end 131.23 111.77) (width 0.2) (layer "F.Cu") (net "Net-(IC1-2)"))
 (segment (start 117.38 115) (end 107.38 125) (width 0.2) (layer "F.Cu") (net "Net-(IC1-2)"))
 (segment (start 130.35 51.46) (end 134.97 56.08) (width 0.2) (layer "F.Cu") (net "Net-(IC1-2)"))
 (segment (start 134.97 56.08) (end 134.97 105.802943) (width 0.2) (layer "F.Cu") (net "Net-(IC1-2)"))
 (segment (start 134.97 105.802943) (end 131.23 109.542943) (width 0.2) (layer "F.Cu") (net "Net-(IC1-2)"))
 (segment (start 128 115) (end 117.38 115) (width 0.2) (layer "F.Cu") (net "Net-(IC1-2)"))
 (segment (start 131.23 111.77) (end 128 115) (width 0.2) (layer "F.Cu") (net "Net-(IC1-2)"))
 (segment (start 125.5 133.69) (end 117.4175 141.7725) (width 0.2) (layer "F.Cu") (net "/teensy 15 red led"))
 (segment (start 88.5925 141.7725) (end 87.06 140.24) (width 0.2) (layer "F.Cu") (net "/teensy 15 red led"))
 (segment (start 117.4175 141.7725) (end 88.5925 141.7725) (width 0.2) (layer "F.Cu") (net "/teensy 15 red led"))
 (segment (start 132.1 141.765635) (end 132.1 111.835) (width 0.2) (layer "B.Cu") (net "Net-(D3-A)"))
 (segment (start 132.1 111.835) (end 129.265 109) (width 0.2) (layer "B.Cu") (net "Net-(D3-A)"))
 (segment (start 131.455635 142.41) (end 132.1 141.765635) (width 0.2) (layer "B.Cu") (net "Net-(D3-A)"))
 (segment (start 125.5 141.31) (end 126.6 142.41) (width 0.2) (layer "B.Cu") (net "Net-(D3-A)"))
 (segment (start 126.6 142.41) (end 131.455635 142.41) (width 0.2) (layer "B.Cu") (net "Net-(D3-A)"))
 (segment (start 131 133.69) (end 122.19 142.5) (width 0.2) (layer "F.Cu") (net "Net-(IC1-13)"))
 (segment (start 122.19 142.5) (end 82 142.5) (width 0.2) (layer "F.Cu") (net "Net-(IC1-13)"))
 (segment (start 81.98 142.48) (end 81.98 140.24) (width 0.2) (layer "F.Cu") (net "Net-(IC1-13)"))
 (segment (start 82 142.5) (end 81.98 142.48) (width 0.2) (layer "F.Cu") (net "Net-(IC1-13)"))
 (segment (start 121 131.31) (end 121 120) (width 0.2) (layer "B.Cu") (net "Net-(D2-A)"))
 (segment (start 121 120) (end 120.765 120) (width 0.2) (layer "B.Cu") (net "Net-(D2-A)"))
 (segment (start 120.765 120) (end 109.765 109) (width 0.2) (layer "B.Cu") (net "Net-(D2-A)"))
 (segment (start 131 141.31) (end 121 131.31) (width 0.2) (layer "B.Cu") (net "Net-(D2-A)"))
 (segment (start 134.17 72.720101) (end 134.17 96.037056) (width 0.2) (layer "F.Cu") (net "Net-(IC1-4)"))
 (segment (start 131.009899 69.56) (end 134.17 72.720101) (width 0.2) (layer "F.Cu") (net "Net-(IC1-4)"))
 (segment (start 112.41 69.56) (end 131.009899 69.56) (width 0.2) (layer "F.Cu") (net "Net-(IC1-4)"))
 (segment (start 103.238404 125) (end 102.3 125) (width 0.2) (layer "F.Cu") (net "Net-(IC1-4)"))
 (segment (start 106.339556 123.8675) (end 104.370903 123.8675) (width 0.2) (layer "F.Cu") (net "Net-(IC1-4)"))
 (segment (start 111.01 70.96) (end 112.41 69.56) (width 0.2) (layer "F.Cu") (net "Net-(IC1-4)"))
 (segment (start 104.370903 123.8675) (end 103.238404 125) (width 0.2) (layer "F.Cu") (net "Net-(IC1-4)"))
 (segment (start 134.17 96.037056) (end 106.339556 123.8675) (width 0.2) (layer "F.Cu") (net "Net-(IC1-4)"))
 (segment (start 82 125) (end 81.98 125) (width 0.2) (layer "B.Cu") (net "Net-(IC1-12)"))
 (segment (start 136.5 133.69) (end 137.6 134.79) (width 0.2) (layer "B.Cu") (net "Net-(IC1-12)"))
 (segment (start 98.3525 140.709097) (end 98.3525 137) (width 0.2) (layer "B.Cu") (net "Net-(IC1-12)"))
 (segment (start 137.6 134.79) (end 137.6 141.765635) (width 0.2) (layer "B.Cu") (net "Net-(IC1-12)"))
 (segment (start 94 137) (end 82 125) (width 0.2) (layer "B.Cu") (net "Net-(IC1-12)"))
 (segment (start 137.6 141.765635) (end 133.465635 145.9) (width 0.2) (layer "B.Cu") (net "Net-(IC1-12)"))
 (segment (start 98.3525 137) (end 94 137) (width 0.2) (layer "B.Cu") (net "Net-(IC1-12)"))
 (segment (start 133.465635 145.9) (end 103.543403 145.9) (width 0.2) (layer "B.Cu") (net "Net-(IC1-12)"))
 (segment (start 103.543403 145.9) (end 98.3525 140.709097) (width 0.2) (layer "B.Cu") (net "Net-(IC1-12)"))
 (segment (start 103 109) (end 118 124) (width 0.2) (layer "B.Cu") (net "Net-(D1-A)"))
 (segment (start 118 124) (end 118 145.5) (width 0.2) (layer "B.Cu") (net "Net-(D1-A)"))
 (segment (start 90 109) (end 103 109) (width 0.2) (layer "B.Cu") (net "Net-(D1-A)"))
 (segment (start 118 145.5) (end 132.31 145.5) (width 0.2) (layer "B.Cu") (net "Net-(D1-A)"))
 (segment (start 132.31 145.5) (end 136.5 141.31) (width 0.2) (layer "B.Cu") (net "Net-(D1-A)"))
 (segment (start 104.42 31) (end 79.04 56.38) (width 0.2) (layer "F.Cu") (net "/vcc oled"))
 (segment (start 79.04 56.38) (end 79.04 127.14) (width 0.2) (layer "F.Cu") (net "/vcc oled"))
 (segment (start 79.04 127.14) (end 81.98 130.08) (width 0.2) (layer "F.Cu") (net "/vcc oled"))
 (segment (start 135.77 53.304315) (end 135.77 117.73) (width 0.2) (layer "F.Cu") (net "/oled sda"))
 (segment (start 135.77 117.73) (end 114.3925 139.1075) (width 0.2) (layer "F.Cu") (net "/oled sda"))
 (segment (start 114.3925 139.1075) (end 95.8125 139.1075) (width 0.2) (layer "F.Cu") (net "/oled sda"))
 (segment (start 95.8125 139.1075) (end 94.68 140.24) (width 0.2) (layer "F.Cu") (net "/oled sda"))
 (segment (start 132.125686 49.66) (end 135.77 53.304315) (width 0.2) (layer "F.Cu") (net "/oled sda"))
 (segment (start 128.16 49.66) (end 132.125686 49.66) (width 0.2) (layer "F.Cu") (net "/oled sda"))
 (segment (start 109.5 31) (end 128.16 49.66) (width 0.2) (layer "F.Cu") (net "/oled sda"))
 (segment (start 93.5475 140.709097) (end 94.210903 141.3725) (width 0.2) (layer "F.Cu") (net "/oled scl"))
 (segment (start 92.5 139) (end 92.6075 139.1075) (width 0.2) (layer "F.Cu") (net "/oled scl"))
 (segment (start 78.5 138.5) (end 79 139) (width 0.2) (layer "F.Cu") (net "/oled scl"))
 (segment (start 95.8125 140.24) (end 97.22 140.24) (width 0.2) (layer "F.Cu") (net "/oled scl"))
 (segment (start 78.64 128.341597) (end 78.5 128.481597) (width 0.2) (layer "F.Cu") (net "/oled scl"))
 (segment (start 92.6075 139.1075) (end 92.609097 139.1075) (width 0.2) (layer "F.Cu") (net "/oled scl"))
 (segment (start 105 27.94) (end 78.64 54.3) (width 0.2) (layer "F.Cu") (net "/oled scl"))
 (segment (start 93.2725 139.7725) (end 93.5475 140.0475) (width 0.2) (layer "F.Cu") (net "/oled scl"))
 (segment (start 92.609097 139.1075) (end 93.2725 139.770903) (width 0.2) (layer "F.Cu") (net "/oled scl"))
 (segment (start 95.8125 140.709097) (end 95.8125 140.24) (width 0.2) (layer "F.Cu") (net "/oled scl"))
 (segment (start 93.2725 139.770903) (end 93.2725 139.7725) (width 0.2) (layer "F.Cu") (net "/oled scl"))
 (segment (start 94.210903 141.3725) (end 95.149097 141.3725) (width 0.2) (layer "F.Cu") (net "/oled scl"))
 (segment (start 79 139) (end 92.5 139) (width 0.2) (layer "F.Cu") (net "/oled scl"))
 (segment (start 93.5475 140.0475) (end 93.5475 140.709097) (width 0.2) (layer "F.Cu") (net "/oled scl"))
 (segment (start 78.5 128.481597) (end 78.5 138.5) (width 0.2) (layer "F.Cu") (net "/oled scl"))
 (segment (start 112.04 31) (end 112.04 30.107208) (width 0.2) (layer "F.Cu") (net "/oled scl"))
 (segment (start 95.149097 141.3725) (end 95.8125 140.709097) (width 0.2) (layer "F.Cu") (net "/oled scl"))
 (segment (start 112.04 30.107208) (end 109.872792 27.94) (width 0.2) (layer "F.Cu") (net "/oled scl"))
 (segment (start 109.872792 27.94) (end 105 27.94) (width 0.2) (layer "F.Cu") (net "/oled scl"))
 (segment (start 78.64 54.3) (end 78.64 128.341597) (width 0.2) (layer "F.Cu") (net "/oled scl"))
 (segment (start 134.57 72.554416) (end 134.57 96.202742) (width 0.2) (layer "F.Cu") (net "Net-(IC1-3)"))
 (segment (start 106.910903 123.8675) (end 105.778403 125) (width 0.2) (layer "F.Cu") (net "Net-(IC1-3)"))
 (segment (start 105.778403 125) (end 104.84 125) (width 0.2) (layer "F.Cu") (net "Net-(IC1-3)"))
 (segment (start 131.175585 69.16) (end 134.57 72.554416) (width 0.2) (layer "F.Cu") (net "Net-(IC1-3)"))
 (segment (start 91.35 70.96) (end 93.15 69.16) (width 0.2) (layer "F.Cu") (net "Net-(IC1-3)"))
 (segment (start 93.15 69.16) (end 131.175585 69.16) (width 0.2) (layer "F.Cu") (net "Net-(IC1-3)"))
 (segment (start 106.910903 123.861839) (end 106.910903 123.8675) (width 0.2) (layer "F.Cu") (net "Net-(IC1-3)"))
 (segment (start 134.57 96.202742) (end 106.910903 123.861839) (width 0.2) (layer "F.Cu") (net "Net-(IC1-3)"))
 (segment (start 110.85 90.46) (end 110.85 98.445635) (width 0.2) (layer "F.Cu") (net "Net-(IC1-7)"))
 (segment (start 91.0075 125.469097) (end 91.670903 126.1325) (width 0.2) (layer "F.Cu") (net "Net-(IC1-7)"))
 (segment (start 91.670903 126.1325) (end 93.5475 126.1325) (width 0.2) (layer "F.Cu") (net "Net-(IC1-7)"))
 (segment (start 91.0075 118.288135) (end 91.0075 125.469097) (width 0.2) (layer "F.Cu") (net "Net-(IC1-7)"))
 (segment (start 93.5475 126.1325) (end 94.68 125) (width 0.2) (layer "F.Cu") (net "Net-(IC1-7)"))
 (segment (start 110.85 98.445635) (end 91.0075 118.288135) (width 0.2) (layer "F.Cu") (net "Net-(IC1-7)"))
 (segment (start 79.44 120.583403) (end 83.3875 124.530903) (width 0.2) (layer "F.Cu") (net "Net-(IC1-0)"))
 (segment (start 89.95 71.539899) (end 79.44 82.049899) (width 0.2) (layer "F.Cu") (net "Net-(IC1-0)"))
 (segment (start 83.3875 124.530903) (end 83.3875 125.469097) (width 0.2) (layer "F.Cu") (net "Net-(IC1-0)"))
 (segment (start 103.46 134) (end 112.46 125) (width 0.2) (layer "F.Cu") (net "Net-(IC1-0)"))
 (segment (start 79.44 82.049899) (end 79.44 120.583403) (width 0.2) (layer "F.Cu") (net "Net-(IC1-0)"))
 (segment (start 91.43 51.46) (end 91.43 68.900101) (width 0.2) (layer "F.Cu") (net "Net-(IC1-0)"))
 (segment (start 83.3875 125.469097) (end 91.918403 134) (width 0.2) (layer "F.Cu") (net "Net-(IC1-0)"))
 (segment (start 91.43 68.900101) (end 89.95 70.380101) (width 0.2) (layer "F.Cu") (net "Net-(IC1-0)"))
 (segment (start 91.918403 134) (end 103.46 134) (width 0.2) (layer "F.Cu") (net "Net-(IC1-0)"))
 (segment (start 89.95 70.380101) (end 89.95 71.539899) (width 0.2) (layer "F.Cu") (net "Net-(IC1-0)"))
 (segment (start 130.43 70.96) (end 130.43 75.197056) (width 0.2) (layer "F.Cu") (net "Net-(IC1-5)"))
 (segment (start 102.945444 123.8675) (end 100.8925 123.8675) (width 0.2) (layer "F.Cu") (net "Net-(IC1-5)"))
 (segment (start 130.43 75.197056) (end 132.472944 77.24) (width 0.2) (layer "F.Cu") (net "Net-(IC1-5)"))
 (segment (start 132.472944 77.24) (end 132.472944 94.34) (width 0.2) (layer "F.Cu") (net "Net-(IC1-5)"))
 (segment (start 132.472944 94.34) (end 102.945444 123.8675) (width 0.2) (layer "F.Cu") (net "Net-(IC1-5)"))
 (segment (start 100.8925 123.8675) (end 99.76 125) (width 0.2) (layer "F.Cu") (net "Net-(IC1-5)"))
 (segment (start 92.14 125) (end 92.14 121.685) (width 0.2) (layer "F.Cu") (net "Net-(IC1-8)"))
 (segment (start 92.14 121.685) (end 123.365 90.46) (width 0.2) (layer "F.Cu") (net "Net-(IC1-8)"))
 (segment (start 123.365 90.46) (end 130.43 90.46) (width 0.2) (layer "F.Cu") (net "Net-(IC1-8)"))
 (segment (start 84.5 119.9) (end 89.6 125) (width 0.2) (layer "F.Cu") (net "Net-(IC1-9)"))
 (segment (start 84.5 96.9) (end 84.5 119.9) (width 0.2) (layer "F.Cu") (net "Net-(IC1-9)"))
 (segment (start 81.14 93.54) (end 84.5 96.9) (width 0.2) (layer "F.Cu") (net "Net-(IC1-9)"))
 (segment (start 81.14 98.54) (end 83.49 100.89) (width 0.2) (layer "F.Cu") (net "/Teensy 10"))
 (segment (start 83.49 121.43) (end 87.06 125) (width 0.2) (layer "F.Cu") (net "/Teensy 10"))
 (segment (start 83.49 100.89) (end 83.49 121.43) (width 0.2) (layer "F.Cu") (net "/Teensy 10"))
 (segment (start 95.64 98.54) (end 89.34 92.24) (width 0.2) (layer "F.Cu") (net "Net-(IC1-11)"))
 (segment (start 79.84 92.24) (end 79.84 120.32) (width 0.2) (layer "F.Cu") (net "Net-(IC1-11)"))
 (segment (start 79.84 120.32) (end 84.52 125) (width 0.2) (layer "F.Cu") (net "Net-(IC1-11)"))
 (segment (start 89.34 92.24) (end 79.84 92.24) (width 0.2) (layer "F.Cu") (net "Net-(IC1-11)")))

